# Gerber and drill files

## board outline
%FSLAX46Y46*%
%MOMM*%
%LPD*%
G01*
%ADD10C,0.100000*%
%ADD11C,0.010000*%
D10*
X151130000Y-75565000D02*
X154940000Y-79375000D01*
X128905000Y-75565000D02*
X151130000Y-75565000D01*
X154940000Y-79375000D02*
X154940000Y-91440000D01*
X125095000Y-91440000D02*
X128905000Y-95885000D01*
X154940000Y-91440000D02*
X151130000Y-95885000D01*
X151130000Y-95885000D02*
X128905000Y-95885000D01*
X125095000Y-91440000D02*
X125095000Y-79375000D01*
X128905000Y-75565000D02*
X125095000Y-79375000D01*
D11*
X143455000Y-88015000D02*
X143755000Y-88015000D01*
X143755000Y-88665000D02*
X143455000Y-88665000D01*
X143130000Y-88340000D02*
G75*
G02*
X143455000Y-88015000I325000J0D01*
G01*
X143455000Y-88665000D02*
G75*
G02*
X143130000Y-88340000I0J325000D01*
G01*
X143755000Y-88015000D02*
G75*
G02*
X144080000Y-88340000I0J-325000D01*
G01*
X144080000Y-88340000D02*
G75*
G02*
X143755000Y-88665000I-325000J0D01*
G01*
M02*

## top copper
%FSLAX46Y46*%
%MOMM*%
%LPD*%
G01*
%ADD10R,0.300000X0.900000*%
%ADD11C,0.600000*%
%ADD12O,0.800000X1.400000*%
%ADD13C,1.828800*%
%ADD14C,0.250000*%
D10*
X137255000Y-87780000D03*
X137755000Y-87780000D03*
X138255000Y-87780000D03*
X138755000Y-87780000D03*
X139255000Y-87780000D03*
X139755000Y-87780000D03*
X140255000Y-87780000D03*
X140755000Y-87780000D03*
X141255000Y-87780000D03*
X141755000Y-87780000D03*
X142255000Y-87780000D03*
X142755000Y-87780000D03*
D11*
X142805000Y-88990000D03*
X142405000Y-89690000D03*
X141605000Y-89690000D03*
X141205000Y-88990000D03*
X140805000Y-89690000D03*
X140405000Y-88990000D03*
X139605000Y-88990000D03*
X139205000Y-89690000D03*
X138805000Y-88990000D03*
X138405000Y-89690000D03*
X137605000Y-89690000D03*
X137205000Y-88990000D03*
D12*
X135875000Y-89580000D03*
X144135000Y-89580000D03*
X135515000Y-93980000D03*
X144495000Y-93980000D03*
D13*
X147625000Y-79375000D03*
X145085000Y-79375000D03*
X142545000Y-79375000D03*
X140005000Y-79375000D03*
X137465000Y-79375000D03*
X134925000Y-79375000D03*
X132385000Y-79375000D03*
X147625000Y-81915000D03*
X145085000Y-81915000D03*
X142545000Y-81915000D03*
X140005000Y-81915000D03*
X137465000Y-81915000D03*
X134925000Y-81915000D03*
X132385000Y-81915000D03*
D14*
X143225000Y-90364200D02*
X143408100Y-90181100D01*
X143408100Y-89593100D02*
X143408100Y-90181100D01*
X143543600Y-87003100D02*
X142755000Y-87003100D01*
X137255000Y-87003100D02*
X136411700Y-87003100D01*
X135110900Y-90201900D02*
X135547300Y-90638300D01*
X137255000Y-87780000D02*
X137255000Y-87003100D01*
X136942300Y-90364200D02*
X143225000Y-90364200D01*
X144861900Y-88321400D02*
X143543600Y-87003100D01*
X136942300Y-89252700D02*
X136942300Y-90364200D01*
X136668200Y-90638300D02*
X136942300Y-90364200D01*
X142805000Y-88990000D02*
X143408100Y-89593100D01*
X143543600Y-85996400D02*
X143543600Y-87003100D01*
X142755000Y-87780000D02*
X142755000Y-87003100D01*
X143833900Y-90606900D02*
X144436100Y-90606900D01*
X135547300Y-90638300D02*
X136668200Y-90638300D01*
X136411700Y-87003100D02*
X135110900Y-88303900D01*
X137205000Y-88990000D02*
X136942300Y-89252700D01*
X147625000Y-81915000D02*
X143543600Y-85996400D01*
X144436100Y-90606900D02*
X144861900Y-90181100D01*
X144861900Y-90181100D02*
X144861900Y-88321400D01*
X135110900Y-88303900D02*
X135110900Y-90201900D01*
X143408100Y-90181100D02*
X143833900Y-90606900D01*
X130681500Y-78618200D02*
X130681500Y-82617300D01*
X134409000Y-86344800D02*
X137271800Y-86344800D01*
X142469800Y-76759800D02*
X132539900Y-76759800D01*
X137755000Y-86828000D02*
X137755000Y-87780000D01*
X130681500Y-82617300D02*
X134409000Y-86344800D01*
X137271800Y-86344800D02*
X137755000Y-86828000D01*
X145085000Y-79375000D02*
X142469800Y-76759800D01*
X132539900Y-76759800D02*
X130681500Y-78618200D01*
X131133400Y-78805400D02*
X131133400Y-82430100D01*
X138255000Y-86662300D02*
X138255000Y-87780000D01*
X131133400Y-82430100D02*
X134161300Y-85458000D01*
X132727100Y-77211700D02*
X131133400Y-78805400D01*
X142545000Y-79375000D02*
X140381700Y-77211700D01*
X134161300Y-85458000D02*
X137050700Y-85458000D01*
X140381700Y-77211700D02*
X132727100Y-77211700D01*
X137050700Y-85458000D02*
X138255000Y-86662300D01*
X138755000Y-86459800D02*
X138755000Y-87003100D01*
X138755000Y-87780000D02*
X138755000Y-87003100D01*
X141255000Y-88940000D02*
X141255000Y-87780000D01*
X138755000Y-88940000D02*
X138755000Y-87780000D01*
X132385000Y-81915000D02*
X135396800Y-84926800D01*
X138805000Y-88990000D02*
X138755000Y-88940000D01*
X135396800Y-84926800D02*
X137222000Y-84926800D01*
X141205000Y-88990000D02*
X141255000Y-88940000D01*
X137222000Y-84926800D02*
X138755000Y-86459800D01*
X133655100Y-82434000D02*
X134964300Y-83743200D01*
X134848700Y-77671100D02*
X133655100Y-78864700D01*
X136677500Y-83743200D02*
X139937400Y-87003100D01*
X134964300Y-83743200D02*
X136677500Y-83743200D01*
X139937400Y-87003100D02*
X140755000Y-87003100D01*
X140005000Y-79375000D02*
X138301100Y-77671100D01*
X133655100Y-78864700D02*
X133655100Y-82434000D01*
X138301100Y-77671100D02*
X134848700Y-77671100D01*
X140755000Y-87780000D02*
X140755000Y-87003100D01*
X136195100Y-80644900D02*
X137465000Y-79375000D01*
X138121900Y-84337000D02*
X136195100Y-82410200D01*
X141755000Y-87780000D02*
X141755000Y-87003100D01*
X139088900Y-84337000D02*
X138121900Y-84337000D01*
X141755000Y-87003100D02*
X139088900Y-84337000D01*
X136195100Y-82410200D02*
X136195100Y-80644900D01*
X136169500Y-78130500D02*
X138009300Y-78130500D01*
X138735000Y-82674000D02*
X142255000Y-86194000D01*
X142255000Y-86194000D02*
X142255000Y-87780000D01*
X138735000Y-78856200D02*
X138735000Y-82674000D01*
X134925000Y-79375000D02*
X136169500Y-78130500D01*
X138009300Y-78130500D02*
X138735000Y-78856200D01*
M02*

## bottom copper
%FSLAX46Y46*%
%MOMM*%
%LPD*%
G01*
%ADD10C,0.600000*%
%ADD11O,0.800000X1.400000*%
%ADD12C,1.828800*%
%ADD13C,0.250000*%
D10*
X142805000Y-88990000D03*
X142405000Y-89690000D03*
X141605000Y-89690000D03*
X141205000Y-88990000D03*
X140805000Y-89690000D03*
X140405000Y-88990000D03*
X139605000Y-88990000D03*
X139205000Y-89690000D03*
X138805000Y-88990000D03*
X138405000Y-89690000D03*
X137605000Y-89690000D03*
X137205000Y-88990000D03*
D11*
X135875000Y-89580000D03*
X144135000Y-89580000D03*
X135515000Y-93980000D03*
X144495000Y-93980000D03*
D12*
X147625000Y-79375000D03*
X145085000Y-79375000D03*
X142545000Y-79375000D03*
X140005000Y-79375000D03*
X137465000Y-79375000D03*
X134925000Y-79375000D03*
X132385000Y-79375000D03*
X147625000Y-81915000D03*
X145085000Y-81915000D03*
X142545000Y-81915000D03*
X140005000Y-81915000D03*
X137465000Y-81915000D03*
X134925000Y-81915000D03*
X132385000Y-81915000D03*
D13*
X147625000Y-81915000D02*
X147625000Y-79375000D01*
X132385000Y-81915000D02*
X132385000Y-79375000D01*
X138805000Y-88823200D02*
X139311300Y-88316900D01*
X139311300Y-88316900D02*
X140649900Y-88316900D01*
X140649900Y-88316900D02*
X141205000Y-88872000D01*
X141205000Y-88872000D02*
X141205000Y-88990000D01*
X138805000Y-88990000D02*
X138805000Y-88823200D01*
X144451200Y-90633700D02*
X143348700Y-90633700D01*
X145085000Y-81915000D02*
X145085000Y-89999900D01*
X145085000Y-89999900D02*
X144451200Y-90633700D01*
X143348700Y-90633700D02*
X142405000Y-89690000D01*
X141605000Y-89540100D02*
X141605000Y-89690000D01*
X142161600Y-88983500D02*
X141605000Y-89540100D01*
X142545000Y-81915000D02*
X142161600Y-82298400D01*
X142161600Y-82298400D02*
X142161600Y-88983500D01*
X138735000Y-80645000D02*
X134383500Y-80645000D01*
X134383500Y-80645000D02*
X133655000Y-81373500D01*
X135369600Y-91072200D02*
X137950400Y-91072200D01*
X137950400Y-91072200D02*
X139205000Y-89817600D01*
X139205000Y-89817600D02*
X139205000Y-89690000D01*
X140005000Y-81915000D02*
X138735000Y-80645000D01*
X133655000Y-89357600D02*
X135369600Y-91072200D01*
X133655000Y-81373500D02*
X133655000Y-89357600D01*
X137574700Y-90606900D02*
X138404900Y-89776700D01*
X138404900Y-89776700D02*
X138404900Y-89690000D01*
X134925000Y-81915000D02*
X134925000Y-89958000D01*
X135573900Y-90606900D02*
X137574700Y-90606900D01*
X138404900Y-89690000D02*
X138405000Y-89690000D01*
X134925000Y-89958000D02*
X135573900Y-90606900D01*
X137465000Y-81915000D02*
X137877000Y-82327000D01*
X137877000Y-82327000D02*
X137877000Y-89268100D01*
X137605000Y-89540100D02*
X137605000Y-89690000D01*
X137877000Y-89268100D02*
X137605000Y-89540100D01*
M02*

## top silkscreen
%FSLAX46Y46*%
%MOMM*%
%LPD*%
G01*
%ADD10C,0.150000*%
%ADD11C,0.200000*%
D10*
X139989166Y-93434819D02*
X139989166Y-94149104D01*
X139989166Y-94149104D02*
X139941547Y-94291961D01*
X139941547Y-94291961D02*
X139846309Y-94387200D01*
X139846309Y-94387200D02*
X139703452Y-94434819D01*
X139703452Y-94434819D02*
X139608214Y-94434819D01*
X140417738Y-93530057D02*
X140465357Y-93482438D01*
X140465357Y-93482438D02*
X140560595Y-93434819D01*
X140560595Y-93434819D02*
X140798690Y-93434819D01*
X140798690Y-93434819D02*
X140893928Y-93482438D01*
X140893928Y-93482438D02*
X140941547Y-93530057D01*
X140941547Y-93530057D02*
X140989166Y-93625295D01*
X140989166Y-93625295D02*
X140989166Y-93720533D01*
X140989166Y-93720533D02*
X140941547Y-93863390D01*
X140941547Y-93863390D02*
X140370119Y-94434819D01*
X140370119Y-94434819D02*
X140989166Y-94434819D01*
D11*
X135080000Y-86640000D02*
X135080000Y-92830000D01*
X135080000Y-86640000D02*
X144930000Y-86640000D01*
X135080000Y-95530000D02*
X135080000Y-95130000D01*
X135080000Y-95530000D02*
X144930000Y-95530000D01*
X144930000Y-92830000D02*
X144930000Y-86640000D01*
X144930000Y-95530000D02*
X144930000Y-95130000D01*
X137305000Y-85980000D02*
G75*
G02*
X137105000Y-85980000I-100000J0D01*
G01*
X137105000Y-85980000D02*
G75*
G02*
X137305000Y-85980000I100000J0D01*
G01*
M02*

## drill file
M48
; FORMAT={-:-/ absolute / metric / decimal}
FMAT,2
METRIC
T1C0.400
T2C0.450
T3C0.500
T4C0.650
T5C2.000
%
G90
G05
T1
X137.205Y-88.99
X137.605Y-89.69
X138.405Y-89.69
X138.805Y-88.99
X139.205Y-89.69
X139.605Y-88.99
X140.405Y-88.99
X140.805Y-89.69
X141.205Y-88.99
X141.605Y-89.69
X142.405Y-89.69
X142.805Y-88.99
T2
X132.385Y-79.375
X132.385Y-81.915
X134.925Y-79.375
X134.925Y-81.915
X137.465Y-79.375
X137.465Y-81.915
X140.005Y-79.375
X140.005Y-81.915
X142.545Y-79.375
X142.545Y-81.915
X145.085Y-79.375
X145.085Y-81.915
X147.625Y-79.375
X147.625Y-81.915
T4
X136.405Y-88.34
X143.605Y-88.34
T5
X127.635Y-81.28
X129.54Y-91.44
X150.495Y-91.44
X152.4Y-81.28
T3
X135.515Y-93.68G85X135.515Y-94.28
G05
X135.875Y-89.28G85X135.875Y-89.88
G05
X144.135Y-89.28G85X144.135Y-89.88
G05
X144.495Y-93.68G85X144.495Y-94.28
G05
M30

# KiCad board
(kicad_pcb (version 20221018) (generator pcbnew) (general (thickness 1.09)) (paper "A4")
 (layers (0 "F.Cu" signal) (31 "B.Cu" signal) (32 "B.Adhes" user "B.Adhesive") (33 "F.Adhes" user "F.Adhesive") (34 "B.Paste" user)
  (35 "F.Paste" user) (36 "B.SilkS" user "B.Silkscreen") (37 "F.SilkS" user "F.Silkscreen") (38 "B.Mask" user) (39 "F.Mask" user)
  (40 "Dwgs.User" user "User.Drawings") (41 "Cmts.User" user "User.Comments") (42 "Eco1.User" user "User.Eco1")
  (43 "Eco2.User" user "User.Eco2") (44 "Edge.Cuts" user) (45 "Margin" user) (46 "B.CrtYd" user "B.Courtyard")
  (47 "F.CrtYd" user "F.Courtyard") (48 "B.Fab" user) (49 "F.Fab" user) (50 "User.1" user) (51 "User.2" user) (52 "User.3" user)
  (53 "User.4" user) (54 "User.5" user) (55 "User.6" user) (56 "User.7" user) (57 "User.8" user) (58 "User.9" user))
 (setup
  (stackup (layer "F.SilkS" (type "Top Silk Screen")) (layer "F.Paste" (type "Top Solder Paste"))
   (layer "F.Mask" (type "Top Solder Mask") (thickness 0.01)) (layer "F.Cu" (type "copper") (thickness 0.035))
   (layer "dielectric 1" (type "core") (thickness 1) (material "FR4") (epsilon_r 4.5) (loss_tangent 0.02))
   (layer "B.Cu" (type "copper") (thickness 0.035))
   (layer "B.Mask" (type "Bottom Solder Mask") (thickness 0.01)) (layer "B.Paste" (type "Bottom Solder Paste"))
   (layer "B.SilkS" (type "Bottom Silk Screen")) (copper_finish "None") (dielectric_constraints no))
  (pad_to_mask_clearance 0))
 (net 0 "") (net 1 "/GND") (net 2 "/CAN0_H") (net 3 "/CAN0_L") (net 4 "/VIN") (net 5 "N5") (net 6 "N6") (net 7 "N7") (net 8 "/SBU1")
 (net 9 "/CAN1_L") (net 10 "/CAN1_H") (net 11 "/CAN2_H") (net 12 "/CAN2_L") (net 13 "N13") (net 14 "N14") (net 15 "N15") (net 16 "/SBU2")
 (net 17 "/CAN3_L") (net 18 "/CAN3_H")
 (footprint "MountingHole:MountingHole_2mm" (layer "F.Cu") (at 152.4 81.28)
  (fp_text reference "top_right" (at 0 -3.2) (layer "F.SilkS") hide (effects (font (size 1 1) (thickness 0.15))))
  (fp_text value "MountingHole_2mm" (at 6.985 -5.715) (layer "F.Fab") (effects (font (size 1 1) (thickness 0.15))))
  (pad "" np_thru_hole circle (at 0 0) (size 2 2) (drill 2) (layers "*.Cu" "*.Mask")))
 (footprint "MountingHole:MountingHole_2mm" (layer "F.Cu") (at 150.495 91.44)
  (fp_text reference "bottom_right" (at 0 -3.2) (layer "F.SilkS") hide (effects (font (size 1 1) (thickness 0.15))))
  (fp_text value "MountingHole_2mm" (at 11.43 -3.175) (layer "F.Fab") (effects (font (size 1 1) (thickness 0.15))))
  (pad "" np_thru_hole circle (at 0 0) (size 2 2) (drill 2) (layers "F&B.Cu" "*.Mask")))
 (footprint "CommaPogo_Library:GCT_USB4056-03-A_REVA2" (layer "F.Cu") (at 140.005 93.98)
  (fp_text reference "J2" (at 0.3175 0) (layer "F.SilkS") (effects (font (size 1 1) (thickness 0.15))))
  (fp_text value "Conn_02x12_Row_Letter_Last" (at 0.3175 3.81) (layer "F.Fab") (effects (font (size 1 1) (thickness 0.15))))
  (fp_line (start -4.925 -7.34) (end -4.925 -1.15) (stroke (width 0.2) (type solid)) (layer "F.SilkS"))
  (fp_line (start -4.925 -7.34) (end 4.925 -7.34) (stroke (width 0.2) (type solid)) (layer "F.SilkS"))
  (fp_line (start -4.925 1.55) (end -4.925 1.15) (stroke (width 0.2) (type solid)) (layer "F.SilkS"))
  (fp_line (start -4.925 1.55) (end 4.925 1.55) (stroke (width 0.2) (type solid)) (layer "F.SilkS"))
  (fp_line (start 4.925 -1.15) (end 4.925 -7.34) (stroke (width 0.2) (type solid)) (layer "F.SilkS"))
  (fp_line (start 4.925 1.55) (end 4.925 1.15) (stroke (width 0.2) (type solid)) (layer "F.SilkS"))
  (fp_circle (center -2.8 -8) (end -2.7 -8) (stroke (width 0.2) (type solid)) (fill none) (layer "F.SilkS"))
  (fp_line (start 3.45 -5.965) (end 3.75 -5.965) (stroke (width 0.01) (type solid)) (layer "Edge.Cuts"))
  (fp_line (start 3.75 -5.315) (end 3.45 -5.315) (stroke (width 0.01) (type solid)) (layer "Edge.Cuts"))
  (fp_arc (start 3.125 -5.64) (mid 3.22019 -5.86981) (end 3.45 -5.965) (stroke (width 0.01) (type solid)) (layer "Edge.Cuts"))
  (fp_arc (start 3.45 -5.315) (mid 3.22019 -5.41019) (end 3.125 -5.64) (stroke (width 0.01) (type solid)) (layer "Edge.Cuts"))
  (fp_arc (start 3.75 -5.965) (mid 3.97981 -5.86981) (end 4.075 -5.64) (stroke (width 0.01) (type solid)) (layer "Edge.Cuts"))
  (fp_arc (start 4.075 -5.64) (mid 3.97981 -5.41019) (end 3.75 -5.315) (stroke (width 0.01) (type solid)) (layer "Edge.Cuts"))
  (pad "" np_thru_hole circle (at -3.6 -5.64) (size 0.65 0.65) (drill 0.65) (layers "*.Cu" "*.Mask"))
  (pad "" np_thru_hole circle (at 3.6 -5.64) (size 0.65 0.65) (drill 0.65) (layers "*.Cu" "*.Mask"))
  (pad "A1" smd rect (at -2.75 -6.2) (size 0.3 0.9) (layers "F.Cu" "F.Paste" "F.Mask") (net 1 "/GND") (solder_mask_margin 0.102))
  (pad "A2" smd rect (at -2.25 -6.2) (size 0.3 0.9) (layers "F.Cu" "F.Paste" "F.Mask") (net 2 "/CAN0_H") (solder_mask_margin 0.102))
  (pad "A3" smd rect (at -1.75 -6.2) (size 0.3 0.9) (layers "F.Cu" "F.Paste" "F.Mask") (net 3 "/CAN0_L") (solder_mask_margin 0.102))
  (pad "A4" smd rect (at -1.25 -6.2) (size 0.3 0.9) (layers "F.Cu" "F.Paste" "F.Mask") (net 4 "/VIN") (solder_mask_margin 0.102))
  (pad "A5" smd rect (at -0.75 -6.2) (size 0.3 0.9) (layers "F.Cu" "F.Paste" "F.Mask") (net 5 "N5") (solder_mask_margin 0.102))
  (pad "A6" smd rect (at -0.25 -6.2) (size 0.3 0.9) (layers "F.Cu" "F.Paste" "F.Mask") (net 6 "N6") (solder_mask_margin 0.102))
  (pad "A7" smd rect (at 0.25 -6.2) (size 0.3 0.9) (layers "F.Cu" "F.Paste" "F.Mask") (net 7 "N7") (solder_mask_margin 0.102))
  (pad "A8" smd rect (at 0.75 -6.2) (size 0.3 0.9) (layers "F.Cu" "F.Paste" "F.Mask") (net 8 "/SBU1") (solder_mask_margin 0.102))
  (pad "A9" smd rect (at 1.25 -6.2) (size 0.3 0.9) (layers "F.Cu" "F.Paste" "F.Mask") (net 4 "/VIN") (solder_mask_margin 0.102))
  (pad "A10" smd rect (at 1.75 -6.2) (size 0.3 0.9) (layers "F.Cu" "F.Paste" "F.Mask") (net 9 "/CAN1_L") (solder_mask_margin 0.102))
  (pad "A11" smd rect (at 2.25 -6.2) (size 0.3 0.9) (layers "F.Cu" "F.Paste" "F.Mask") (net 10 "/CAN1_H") (solder_mask_margin 0.102))
  (pad "A12" smd rect (at 2.75 -6.2) (size 0.3 0.9) (layers "F.Cu" "F.Paste" "F.Mask") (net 1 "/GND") (solder_mask_margin 0.102))
  (pad "B1" thru_hole circle (at 2.8 -4.99) (size 0.6 0.6) (drill 0.4) (layers "*.Cu" "*.Mask") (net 1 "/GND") (solder_mask_margin 0.102))
  (pad "B2" thru_hole circle (at 2.4 -4.29) (size 0.6 0.6) (drill 0.4) (layers "*.Cu" "*.Mask") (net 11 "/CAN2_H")
   (solder_mask_margin 0.102))
  (pad "B3" thru_hole circle (at 1.6 -4.29) (size 0.6 0.6) (drill 0.4) (layers "*.Cu" "*.Mask") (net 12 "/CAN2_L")
   (solder_mask_margin 0.102))
  (pad "B4" thru_hole circle (at 1.2 -4.99) (size 0.6 0.6) (drill 0.4) (layers "*.Cu" "*.Mask") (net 4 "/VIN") (solder_mask_margin 0.102))
  (pad "B5" thru_hole circle (at 0.8 -4.29) (size 0.6 0.6) (drill 0.4) (layers "*.Cu" "*.Mask") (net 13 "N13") (solder_mask_margin 0.102))
  (pad "B6" thru_hole circle (at 0.4 -4.99) (size 0.6 0.6) (drill 0.4) (layers "*.Cu" "*.Mask") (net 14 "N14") (solder_mask_margin 0.102))
  (pad "B7" thru_hole circle (at -0.4 -4.99) (size 0.6 0.6) (drill 0.4) (layers "*.Cu" "*.Mask") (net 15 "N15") (solder_mask_margin 0.102))
  (pad "B8" thru_hole circle (at -0.8 -4.29) (size 0.6 0.6) (drill 0.4) (layers "*.Cu" "*.Mask") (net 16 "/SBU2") (solder_mask_margin 0.102))
  (pad "B9" thru_hole circle (at -1.2 -4.99) (size 0.6 0.6) (drill 0.4) (layers "*.Cu" "*.Mask") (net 4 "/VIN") (solder_mask_margin 0.102))
  (pad "B10" thru_hole circle (at -1.6 -4.29) (size 0.6 0.6) (drill 0.4) (layers "*.Cu" "*.Mask") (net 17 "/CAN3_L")
   (solder_mask_margin 0.102))
  (pad "B11" thru_hole circle (at -2.4 -4.29) (size 0.6 0.6) (drill 0.4) (layers "*.Cu" "*.Mask") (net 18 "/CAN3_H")
   (solder_mask_margin 0.102))
  (pad "B12" thru_hole circle (at -2.8 -4.99) (size 0.6 0.6) (drill 0.4) (layers "*.Cu" "*.Mask") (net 1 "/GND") (solder_mask_margin 0.102))
  (pad "S1" thru_hole oval (at -4.13 -4.4) (size 0.8 1.4) (drill oval 0.5 1.1) (layers "*.Cu" "*.Mask") (solder_mask_margin 0.102))
  (pad "S2" thru_hole oval (at 4.13 -4.4) (size 0.8 1.4) (drill oval 0.5 1.1) (layers "*.Cu" "*.Mask") (solder_mask_margin 0.102))
  (pad "S3" thru_hole oval (at -4.49 0) (size 0.8 1.4) (drill oval 0.5 1.1) (layers "*.Cu" "*.Mask") (solder_mask_margin 0.102))
  (pad "S4" thru_hole oval (at 4.49 0) (size 0.8 1.4) (drill oval 0.5 1.1) (layers "*.Cu" "*.Mask") (solder_mask_margin 0.102)))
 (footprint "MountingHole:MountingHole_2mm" (layer "F.Cu") (at 127.635 81.28)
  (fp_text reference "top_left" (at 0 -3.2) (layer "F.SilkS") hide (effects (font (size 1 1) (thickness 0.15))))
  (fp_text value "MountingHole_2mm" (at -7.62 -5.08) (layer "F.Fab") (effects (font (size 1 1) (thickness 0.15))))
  (pad "" np_thru_hole circle (at 0 0) (size 2 2) (drill 2) (layers "*.Cu" "*.Mask")))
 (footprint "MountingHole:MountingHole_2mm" (layer "F.Cu") (at 129.54 91.44)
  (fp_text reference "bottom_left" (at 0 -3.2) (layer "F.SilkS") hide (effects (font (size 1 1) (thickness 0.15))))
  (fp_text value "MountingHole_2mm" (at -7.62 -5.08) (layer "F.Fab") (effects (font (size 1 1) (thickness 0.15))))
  (pad "" np_thru_hole circle (at 0 0) (size 2 2) (drill 2) (layers "F&B.Cu" "*.Mask")))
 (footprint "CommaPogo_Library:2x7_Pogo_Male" (layer "B.Cu") (at 140.005 83.82 180)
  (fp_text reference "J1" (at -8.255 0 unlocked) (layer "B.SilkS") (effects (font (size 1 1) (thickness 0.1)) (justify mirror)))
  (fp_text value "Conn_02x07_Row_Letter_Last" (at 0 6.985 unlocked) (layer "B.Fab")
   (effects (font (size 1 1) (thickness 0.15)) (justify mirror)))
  (pad "1" thru_hole circle (at -7.62 4.445 180) (size 1.8288 1.8288) (drill 0.45) (layers "*.Cu" "*.Mask") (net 1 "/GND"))
  (pad "2" thru_hole circle (at -5.08 4.445 180) (size 1.8288 1.8288) (drill 0.45) (layers "*.Cu" "*.Mask") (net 2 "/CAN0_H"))
  (pad "3" thru_hole circle (at -2.54 4.445 180) (size 1.8288 1.8288) (drill 0.45) (layers "*.Cu" "*.Mask") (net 3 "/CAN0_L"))
  (pad "4" thru_hole circle (at 0 4.445 180) (size 1.8288 1.8288) (drill 0.45) (layers "*.Cu" "*.Mask") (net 8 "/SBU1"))
  (pad "5" thru_hole circle (at 2.54 4.445 180) (size 1.8288 1.8288) (drill 0.45) (layers "*.Cu" "*.Mask") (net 9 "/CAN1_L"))
  (pad "6" thru_hole circle (at 5.08 4.445 180) (size 1.8288 1.8288) (drill 0.45) (layers "*.Cu" "*.Mask") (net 10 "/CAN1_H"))
  (pad "7" thru_hole circle (at 7.62 4.445 180) (size 1.8288 1.8288) (drill 0.45) (layers "*.Cu" "*.Mask") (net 4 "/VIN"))
  (pad "8" thru_hole circle (at -7.62 1.905 180) (size 1.8288 1.8288) (drill 0.45) (layers "*.Cu" "*.Mask") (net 1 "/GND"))
  (pad "9" thru_hole circle (at -5.08 1.905 180) (size 1.8288 1.8288) (drill 0.45) (layers "*.Cu" "*.Mask") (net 11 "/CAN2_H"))
  (pad "10" thru_hole circle (at -2.54 1.905 180) (size 1.8288 1.8288) (drill 0.45) (layers "*.Cu" "*.Mask") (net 12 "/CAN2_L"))
  (pad "11" thru_hole circle (at 0 1.905 180) (size 1.8288 1.8288) (drill 0.45) (layers "*.Cu" "*.Mask") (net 16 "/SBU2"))
  (pad "12" thru_hole circle (at 2.54 1.905 180) (size 1.8288 1.8288) (drill 0.45) (layers "*.Cu" "*.Mask") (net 18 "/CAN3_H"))
  (pad "13" thru_hole circle (at 5.08 1.905 180) (size 1.8288 1.8288) (drill 0.45) (layers "*.Cu" "*.Mask") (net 17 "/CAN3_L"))
  (pad "14" thru_hole circle (at 7.62 1.905 180) (size 1.8288 1.8288) (drill 0.45) (layers "*.Cu" "*.Mask") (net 4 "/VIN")))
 (gr_line (start 151.13 75.565) (end 154.94 79.375) (stroke (width 0.1) (type default)) (layer "Edge.Cuts"))
 (gr_line (start 128.905 75.565) (end 151.13 75.565) (stroke (width 0.1) (type default)) (layer "Edge.Cuts"))
 (gr_line (start 154.94 79.375) (end 154.94 91.44) (stroke (width 0.1) (type default)) (layer "Edge.Cuts"))
 (gr_line (start 125.095 91.44) (end 128.905 95.885) (stroke (width 0.1) (type default)) (layer "Edge.Cuts"))
 (gr_line (start 154.94 91.44) (end 151.13 95.885) (stroke (width 0.1) (type default)) (layer "Edge.Cuts"))
 (gr_line (start 151.13 95.885) (end 128.905 95.885) (stroke (width 0.1) (type default)) (layer "Edge.Cuts"))
 (gr_line (start 125.095 91.44) (end 125.095 79.375) (stroke (width 0.1) (type default)) (layer "Edge.Cuts"))
 (gr_line (start 128.905 75.565) (end 125.095 79.375) (stroke (width 0.1) (type default)) (layer "Edge.Cuts"))
 (segment (start 143.225 90.3642) (end 143.4081 90.1811) (width 0.25) (layer "F.Cu") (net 1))
 (segment (start 143.4081 89.5931) (end 143.4081 90.1811) (width 0.25) (layer "F.Cu") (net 1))
 (segment (start 143.5436 87.0031) (end 142.755 87.0031) (width 0.25) (layer "F.Cu") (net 1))
 (segment (start 137.255 87.0031) (end 136.4117 87.0031) (width 0.25) (layer "F.Cu") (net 1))
 (segment (start 135.1109 90.2019) (end 135.5473 90.6383) (width 0.25) (layer "F.Cu") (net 1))
 (segment (start 137.255 87.78) (end 137.255 87.0031) (width 0.25) (layer "F.Cu") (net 1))
 (segment (start 136.9423 90.3642) (end 143.225 90.3642) (width 0.25) (layer "F.Cu") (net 1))
 (segment (start 144.8619 88.3214) (end 143.5436 87.0031) (width 0.25) (layer "F.Cu") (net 1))
 (segment (start 136.9423 89.2527) (end 136.9423 90.3642) (width 0.25) (layer "F.Cu") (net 1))
 (segment (start 136.6682 90.6383) (end 136.9423 90.3642) (width 0.25) (layer "F.Cu") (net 1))
 (segment (start 142.805 88.99) (end 143.4081 89.5931) (width 0.25) (layer "F.Cu") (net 1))
 (segment (start 143.5436 85.9964) (end 143.5436 87.0031) (width 0.25) (layer "F.Cu") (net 1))
 (segment (start 142.755 87.78) (end 142.755 87.0031) (width 0.25) (layer "F.Cu") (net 1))
 (segment (start 143.8339 90.6069) (end 144.4361 90.6069) (width 0.25) (layer "F.Cu") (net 1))
 (segment (start 135.5473 90.6383) (end 136.6682 90.6383) (width 0.25) (layer "F.Cu") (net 1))
 (segment (start 136.4117 87.0031) (end 135.1109 88.3039) (width 0.25) (layer "F.Cu") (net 1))
 (segment (start 137.205 88.99) (end 136.9423 89.2527) (width 0.25) (layer "F.Cu") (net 1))
 (segment (start 147.625 81.915) (end 143.5436 85.9964) (width 0.25) (layer "F.Cu") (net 1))
 (segment (start 144.4361 90.6069) (end 144.8619 90.1811) (width 0.25) (layer "F.Cu") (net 1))
 (segment (start 144.8619 90.1811) (end 144.8619 88.3214) (width 0.25) (layer "F.Cu") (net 1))
 (segment (start 135.1109 88.3039) (end 135.1109 90.2019) (width 0.25) (layer "F.Cu") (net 1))
 (segment (start 143.4081 90.1811) (end 143.8339 90.6069) (width 0.25) (layer "F.Cu") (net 1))
 (segment (start 147.625 81.915) (end 147.625 79.375) (width 0.25) (layer "B.Cu") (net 1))
 (segment (start 130.6815 78.6182) (end 130.6815 82.6173) (width 0.25) (layer "F.Cu") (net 2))
 (segment (start 134.409 86.3448) (end 137.2718 86.3448) (width 0.25) (layer "F.Cu") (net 2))
 (segment (start 142.4698 76.7598) (end 132.5399 76.7598) (width 0.25) (layer "F.Cu") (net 2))
 (segment (start 137.755 86.828) (end 137.755 87.78) (width 0.25) (layer "F.Cu") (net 2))
 (segment (start 130.6815 82.6173) (end 134.409 86.3448) (width 0.25) (layer "F.Cu") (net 2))
 (segment (start 137.2718 86.3448) (end 137.755 86.828) (width 0.25) (layer "F.Cu") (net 2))
 (segment (start 145.085 79.375) (end 142.4698 76.7598) (width 0.25) (layer "F.Cu") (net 2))
 (segment (start 132.5399 76.7598) (end 130.6815 78.6182) (width 0.25) (layer "F.Cu") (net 2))
 (segment (start 131.1334 78.8054) (end 131.1334 82.4301) (width 0.25) (layer "F.Cu") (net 3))
 (segment (start 138.255 86.6623) (end 138.255 87.78) (width 0.25) (layer "F.Cu") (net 3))
 (segment (start 131.1334 82.4301) (end 134.1613 85.458) (width 0.25) (layer "F.Cu") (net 3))
 (segment (start 132.7271 77.2117) (end 131.1334 78.8054) (width 0.25) (layer "F.Cu") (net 3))
 (segment (start 142.545 79.375) (end 140.3817 77.2117) (width 0.25) (layer "F.Cu") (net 3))
 (segment (start 134.1613 85.458) (end 137.0507 85.458) (width 0.25) (layer "F.Cu") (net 3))
 (segment (start 140.3817 77.2117) (end 132.7271 77.2117) (width 0.25) (layer "F.Cu") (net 3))
 (segment (start 137.0507 85.458) (end 138.255 86.6623) (width 0.25) (layer "F.Cu") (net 3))
 (segment (start 138.755 86.4598) (end 138.755 87.0031) (width 0.25) (layer "F.Cu") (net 4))
 (segment (start 138.755 87.78) (end 138.755 87.0031) (width 0.25) (layer "F.Cu") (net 4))
 (segment (start 141.255 88.94) (end 141.255 87.78) (width 0.25) (layer "F.Cu") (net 4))
 (segment (start 138.755 88.94) (end 138.755 87.78) (width 0.25) (layer "F.Cu") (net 4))
 (segment (start 132.385 81.915) (end 135.3968 84.9268) (width 0.25) (layer "F.Cu") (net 4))
 (segment (start 138.805 88.99) (end 138.755 88.94) (width 0.25) (layer "F.Cu") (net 4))
 (segment (start 135.3968 84.9268) (end 137.222 84.9268) (width 0.25) (layer "F.Cu") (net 4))
 (segment (start 141.205 88.99) (end 141.255 88.94) (width 0.25) (layer "F.Cu") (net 4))
 (segment (start 137.222 84.9268) (end 138.755 86.4598) (width 0.25) (layer "F.Cu") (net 4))
 (segment (start 132.385 81.915) (end 132.385 79.375) (width 0.25) (layer "B.Cu") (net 4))
 (segment (start 138.805 88.8232) (end 139.3113 88.3169) (width 0.25) (layer "B.Cu") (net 4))
 (segment (start 139.3113 88.3169) (end 140.6499 88.3169) (width 0.25) (layer "B.Cu") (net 4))
 (segment (start 140.6499 88.3169) (end 141.205 88.872) (width 0.25) (layer "B.Cu") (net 4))
 (segment (start 141.205 88.872) (end 141.205 88.99) (width 0.25) (layer "B.Cu") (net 4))
 (segment (start 138.805 88.99) (end 138.805 88.8232) (width 0.25) (layer "B.Cu") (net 4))
 (segment (start 133.6551 82.434) (end 134.9643 83.7432) (width 0.25) (layer "F.Cu") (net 8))
 (segment (start 134.8487 77.6711) (end 133.6551 78.8647) (width 0.25) (layer "F.Cu") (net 8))
 (segment (start 136.6775 83.7432) (end 139.9374 87.0031) (width 0.25) (layer "F.Cu") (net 8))
 (segment (start 134.9643 83.7432) (end 136.6775 83.7432) (width 0.25) (layer "F.Cu") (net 8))
 (segment (start 139.9374 87.0031) (end 140.755 87.0031) (width 0.25) (layer "F.Cu") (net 8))
 (segment (start 140.005 79.375) (end 138.3011 77.6711) (width 0.25) (layer "F.Cu") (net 8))
 (segment (start 133.6551 78.8647) (end 133.6551 82.434) (width 0.25) (layer "F.Cu") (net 8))
 (segment (start 138.3011 77.6711) (end 134.8487 77.6711) (width 0.25) (layer "F.Cu") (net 8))
 (segment (start 140.755 87.78) (end 140.755 87.0031) (width 0.25) (layer "F.Cu") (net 8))
 (segment (start 136.1951 80.6449) (end 137.465 79.375) (width 0.25) (layer "F.Cu") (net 9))
 (segment (start 138.1219 84.337) (end 136.1951 82.4102) (width 0.25) (layer "F.Cu") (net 9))
 (segment (start 141.755 87.78) (end 141.755 87.0031) (width 0.25) (layer "F.Cu") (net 9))
 (segment (start 139.0889 84.337) (end 138.1219 84.337) (width 0.25) (layer "F.Cu") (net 9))
 (segment (start 141.755 87.0031) (end 139.0889 84.337) (width 0.25) (layer "F.Cu") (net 9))
 (segment (start 136.1951 82.4102) (end 136.1951 80.6449) (width 0.25) (layer "F.Cu") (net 9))
 (segment (start 136.1695 78.1305) (end 138.0093 78.1305) (width 0.25) (layer "F.Cu") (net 10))
 (segment (start 138.735 82.674) (end 142.255 86.194) (width 0.25) (layer "F.Cu") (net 10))
 (segment (start 142.255 86.194) (end 142.255 87.78) (width 0.25) (layer "F.Cu") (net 10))
 (segment (start 138.735 78.8562) (end 138.735 82.674) (width 0.25) (layer "F.Cu") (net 10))
 (segment (start 134.925 79.375) (end 136.1695 78.1305) (width 0.25) (layer "F.Cu") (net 10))
 (segment (start 138.0093 78.1305) (end 138.735 78.8562) (width 0.25) (layer "F.Cu") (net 10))
 (segment (start 144.4512 90.6337) (end 143.3487 90.6337) (width 0.25) (layer "B.Cu") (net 11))
 (segment (start 145.085 81.915) (end 145.085 89.9999) (width 0.25) (layer "B.Cu") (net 11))
 (segment (start 145.085 89.9999) (end 144.4512 90.6337) (width 0.25) (layer "B.Cu") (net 11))
 (segment (start 143.3487 90.6337) (end 142.405 89.69) (width 0.25) (layer "B.Cu") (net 11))
 (segment (start 141.605 89.5401) (end 141.605 89.69) (width 0.25) (layer "B.Cu") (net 12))
 (segment (start 142.1616 88.9835) (end 141.605 89.5401) (width 0.25) (layer "B.Cu") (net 12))
 (segment (start 142.545 81.915) (end 142.1616 82.2984) (width 0.25) (layer "B.Cu") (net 12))
 (segment (start 142.1616 82.2984) (end 142.1616 88.9835) (width 0.25) (layer "B.Cu") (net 12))
 (segment (start 138.735 80.645) (end 134.3835 80.645) (width 0.25) (layer "B.Cu") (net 16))
 (segment (start 134.3835 80.645) (end 133.655 81.3735) (width 0.25) (layer "B.Cu") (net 16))
 (segment (start 135.3696 91.0722) (end 137.9504 91.0722) (width 0.25) (layer "B.Cu") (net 16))
 (segment (start 137.9504 91.0722) (end 139.205 89.8176) (width 0.25) (layer "B.Cu") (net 16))
 (segment (start 139.205 89.8176) (end 139.205 89.69) (width 0.25) (layer "B.Cu") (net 16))
 (segment (start 140.005 81.915) (end 138.735 80.645) (width 0.25) (layer "B.Cu") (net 16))
 (segment (start 133.655 89.3576) (end 135.3696 91.0722) (width 0.25) (layer "B.Cu") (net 16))
 (segment (start 133.655 81.3735) (end 133.655 89.3576) (width 0.25) (layer "B.Cu") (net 16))
 (segment (start 137.5747 90.6069) (end 138.4049 89.7767) (width 0.25) (layer "B.Cu") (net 17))
 (segment (start 138.4049 89.7767) (end 138.4049 89.69) (width 0.25) (layer "B.Cu") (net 17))
 (segment (start 134.925 81.915) (end 134.925 89.958) (width 0.25) (layer "B.Cu") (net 17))
 (segment (start 135.5739 90.6069) (end 137.5747 90.6069) (width 0.25) (layer "B.Cu") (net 17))
 (segment (start 138.4049 89.69) (end 138.405 89.69) (width 0.25) (layer "B.Cu") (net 17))
 (segment (start 134.925 89.958) (end 135.5739 90.6069) (width 0.25) (layer "B.Cu") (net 17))
 (segment (start 137.465 81.915) (end 137.877 82.327) (width 0.25) (layer "B.Cu") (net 18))
 (segment (start 137.877 82.327) (end 137.877 89.2681) (width 0.25) (layer "B.Cu") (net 18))
 (segment (start 137.605 89.5401) (end 137.605 89.69) (width 0.25) (layer "B.Cu") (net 18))
 (segment (start 137.877 89.2681) (end 137.605 89.5401) (width 0.25) (layer "B.Cu") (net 18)))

